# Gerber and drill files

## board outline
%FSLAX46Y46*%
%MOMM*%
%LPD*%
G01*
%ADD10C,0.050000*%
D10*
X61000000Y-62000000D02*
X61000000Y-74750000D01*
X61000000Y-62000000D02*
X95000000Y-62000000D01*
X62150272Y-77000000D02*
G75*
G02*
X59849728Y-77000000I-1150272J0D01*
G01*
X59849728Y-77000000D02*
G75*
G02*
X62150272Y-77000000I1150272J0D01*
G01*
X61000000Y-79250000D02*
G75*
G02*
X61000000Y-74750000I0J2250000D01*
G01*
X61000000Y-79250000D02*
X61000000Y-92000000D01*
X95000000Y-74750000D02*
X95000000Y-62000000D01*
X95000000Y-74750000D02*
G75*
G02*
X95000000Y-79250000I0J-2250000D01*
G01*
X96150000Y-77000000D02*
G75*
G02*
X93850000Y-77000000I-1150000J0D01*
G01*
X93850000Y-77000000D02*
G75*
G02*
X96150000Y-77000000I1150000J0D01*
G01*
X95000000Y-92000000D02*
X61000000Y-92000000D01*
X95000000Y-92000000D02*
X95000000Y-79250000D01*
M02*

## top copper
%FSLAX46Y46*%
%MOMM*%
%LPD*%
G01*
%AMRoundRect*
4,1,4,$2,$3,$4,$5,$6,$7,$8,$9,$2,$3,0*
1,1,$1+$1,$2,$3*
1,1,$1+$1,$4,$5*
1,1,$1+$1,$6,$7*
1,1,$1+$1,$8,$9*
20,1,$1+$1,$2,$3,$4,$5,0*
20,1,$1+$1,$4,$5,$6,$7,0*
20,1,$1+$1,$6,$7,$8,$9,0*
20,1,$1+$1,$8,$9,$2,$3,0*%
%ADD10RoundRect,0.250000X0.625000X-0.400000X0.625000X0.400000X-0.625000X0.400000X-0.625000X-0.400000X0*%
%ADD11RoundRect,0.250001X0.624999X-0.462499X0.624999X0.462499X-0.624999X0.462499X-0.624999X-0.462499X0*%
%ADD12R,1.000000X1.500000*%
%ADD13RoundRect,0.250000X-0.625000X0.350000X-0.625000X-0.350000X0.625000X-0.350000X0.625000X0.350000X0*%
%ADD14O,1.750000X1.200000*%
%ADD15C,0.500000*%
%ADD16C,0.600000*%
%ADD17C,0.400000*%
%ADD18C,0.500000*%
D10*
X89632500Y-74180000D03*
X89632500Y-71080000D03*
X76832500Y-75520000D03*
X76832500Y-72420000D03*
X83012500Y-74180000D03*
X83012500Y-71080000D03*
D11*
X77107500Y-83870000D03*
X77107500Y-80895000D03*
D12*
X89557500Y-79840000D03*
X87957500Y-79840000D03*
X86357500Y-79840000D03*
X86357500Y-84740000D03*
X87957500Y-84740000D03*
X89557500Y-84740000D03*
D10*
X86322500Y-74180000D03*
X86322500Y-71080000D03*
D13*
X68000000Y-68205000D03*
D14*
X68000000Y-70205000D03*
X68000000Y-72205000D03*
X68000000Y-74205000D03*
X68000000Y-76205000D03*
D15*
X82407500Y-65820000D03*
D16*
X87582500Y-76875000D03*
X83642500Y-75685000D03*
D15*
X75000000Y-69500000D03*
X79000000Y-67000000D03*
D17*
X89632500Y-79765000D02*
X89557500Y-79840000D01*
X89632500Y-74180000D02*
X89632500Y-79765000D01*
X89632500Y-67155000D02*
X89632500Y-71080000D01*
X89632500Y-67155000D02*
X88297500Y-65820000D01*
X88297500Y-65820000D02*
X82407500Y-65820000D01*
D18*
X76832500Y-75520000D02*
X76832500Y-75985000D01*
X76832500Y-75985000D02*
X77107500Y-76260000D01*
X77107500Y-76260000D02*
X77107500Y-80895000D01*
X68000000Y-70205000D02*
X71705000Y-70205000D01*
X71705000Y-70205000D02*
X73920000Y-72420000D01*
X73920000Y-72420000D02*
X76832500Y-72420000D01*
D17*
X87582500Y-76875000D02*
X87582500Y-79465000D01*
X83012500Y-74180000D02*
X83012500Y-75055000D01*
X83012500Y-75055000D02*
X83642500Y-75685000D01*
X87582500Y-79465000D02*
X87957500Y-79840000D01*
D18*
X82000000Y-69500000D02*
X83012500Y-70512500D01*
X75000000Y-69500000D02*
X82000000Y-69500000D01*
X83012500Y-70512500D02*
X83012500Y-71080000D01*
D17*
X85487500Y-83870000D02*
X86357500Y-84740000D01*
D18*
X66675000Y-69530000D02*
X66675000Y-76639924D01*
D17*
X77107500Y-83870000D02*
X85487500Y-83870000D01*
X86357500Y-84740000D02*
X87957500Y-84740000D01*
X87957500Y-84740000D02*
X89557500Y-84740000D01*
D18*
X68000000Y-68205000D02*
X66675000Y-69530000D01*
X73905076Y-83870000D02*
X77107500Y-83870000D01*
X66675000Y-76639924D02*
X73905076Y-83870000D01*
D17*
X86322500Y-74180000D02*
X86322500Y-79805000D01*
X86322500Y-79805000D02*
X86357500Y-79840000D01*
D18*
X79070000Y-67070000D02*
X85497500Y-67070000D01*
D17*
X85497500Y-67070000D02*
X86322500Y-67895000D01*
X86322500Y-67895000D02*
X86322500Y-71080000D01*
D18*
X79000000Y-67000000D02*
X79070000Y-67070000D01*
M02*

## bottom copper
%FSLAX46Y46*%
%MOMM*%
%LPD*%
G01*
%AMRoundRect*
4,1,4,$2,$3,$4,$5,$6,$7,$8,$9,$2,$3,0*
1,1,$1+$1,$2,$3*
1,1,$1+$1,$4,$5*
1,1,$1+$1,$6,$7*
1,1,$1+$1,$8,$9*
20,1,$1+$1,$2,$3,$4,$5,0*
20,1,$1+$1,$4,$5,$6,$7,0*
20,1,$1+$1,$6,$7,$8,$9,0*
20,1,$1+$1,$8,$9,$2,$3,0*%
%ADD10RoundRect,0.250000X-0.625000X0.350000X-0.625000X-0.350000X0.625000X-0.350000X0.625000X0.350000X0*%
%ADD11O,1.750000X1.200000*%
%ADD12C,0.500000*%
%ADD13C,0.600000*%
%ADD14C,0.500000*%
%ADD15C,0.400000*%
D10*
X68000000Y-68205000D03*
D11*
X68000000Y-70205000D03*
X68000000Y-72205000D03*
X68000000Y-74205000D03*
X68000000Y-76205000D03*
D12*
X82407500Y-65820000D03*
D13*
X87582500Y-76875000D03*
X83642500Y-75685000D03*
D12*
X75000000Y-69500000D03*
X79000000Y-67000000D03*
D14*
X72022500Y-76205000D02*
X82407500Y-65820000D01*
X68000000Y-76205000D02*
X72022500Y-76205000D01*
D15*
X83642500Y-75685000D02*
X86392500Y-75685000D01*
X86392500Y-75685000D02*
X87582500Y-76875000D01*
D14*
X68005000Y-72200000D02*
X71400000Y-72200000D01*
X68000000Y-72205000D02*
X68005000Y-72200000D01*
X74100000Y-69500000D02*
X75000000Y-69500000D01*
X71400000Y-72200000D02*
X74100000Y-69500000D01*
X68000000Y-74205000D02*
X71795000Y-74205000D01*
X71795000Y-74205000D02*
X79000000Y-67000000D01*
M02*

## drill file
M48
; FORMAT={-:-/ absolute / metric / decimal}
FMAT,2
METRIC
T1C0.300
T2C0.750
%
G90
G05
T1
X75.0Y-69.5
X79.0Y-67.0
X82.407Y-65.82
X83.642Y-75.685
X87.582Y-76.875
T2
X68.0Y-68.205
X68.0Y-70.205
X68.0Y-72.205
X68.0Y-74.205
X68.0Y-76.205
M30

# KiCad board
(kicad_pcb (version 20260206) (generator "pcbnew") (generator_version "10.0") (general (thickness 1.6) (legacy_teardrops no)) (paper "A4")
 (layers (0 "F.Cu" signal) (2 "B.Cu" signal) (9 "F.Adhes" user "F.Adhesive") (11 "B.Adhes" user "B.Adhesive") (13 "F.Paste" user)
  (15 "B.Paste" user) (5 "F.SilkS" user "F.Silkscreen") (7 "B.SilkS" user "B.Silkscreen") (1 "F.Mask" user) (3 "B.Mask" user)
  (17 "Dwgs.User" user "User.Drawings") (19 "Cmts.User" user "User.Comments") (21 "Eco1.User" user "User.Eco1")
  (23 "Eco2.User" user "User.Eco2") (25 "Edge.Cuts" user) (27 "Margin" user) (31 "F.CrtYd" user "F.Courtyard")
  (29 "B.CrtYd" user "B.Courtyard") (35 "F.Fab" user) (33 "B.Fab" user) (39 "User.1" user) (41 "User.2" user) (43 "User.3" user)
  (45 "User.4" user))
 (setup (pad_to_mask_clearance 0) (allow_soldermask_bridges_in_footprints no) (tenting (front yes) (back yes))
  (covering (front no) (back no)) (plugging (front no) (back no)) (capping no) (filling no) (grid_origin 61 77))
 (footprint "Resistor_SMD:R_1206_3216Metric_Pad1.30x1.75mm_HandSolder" (layer "F.Cu") (at 89.6325 72.63 90)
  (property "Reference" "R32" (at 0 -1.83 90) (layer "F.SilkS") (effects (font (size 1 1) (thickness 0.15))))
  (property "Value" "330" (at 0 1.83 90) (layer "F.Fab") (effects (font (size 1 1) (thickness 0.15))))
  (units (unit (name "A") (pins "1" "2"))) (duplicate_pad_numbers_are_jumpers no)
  (pad "1" smd roundrect (at -1.55 0 90) (size 1.3 1.75) (layers "F.Cu" "F.Mask" "F.Paste") (roundrect_rratio 0.192308)
   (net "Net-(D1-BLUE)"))
  (pad "2" smd roundrect (at 1.55 0 90) (size 1.3 1.75) (layers "F.Cu" "F.Mask" "F.Paste") (roundrect_rratio 0.192308) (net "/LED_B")))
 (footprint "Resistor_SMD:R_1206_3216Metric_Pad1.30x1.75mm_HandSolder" (layer "F.Cu") (at 76.8325 73.97 90)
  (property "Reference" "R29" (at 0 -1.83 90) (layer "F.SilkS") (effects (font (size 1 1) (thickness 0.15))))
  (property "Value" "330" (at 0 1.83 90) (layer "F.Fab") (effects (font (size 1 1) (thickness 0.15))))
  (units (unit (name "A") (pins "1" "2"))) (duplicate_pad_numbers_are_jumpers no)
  (pad "1" smd roundrect (at -1.55 0 90) (size 1.3 1.75) (layers "F.Cu" "F.Mask" "F.Paste") (roundrect_rratio 0.192308) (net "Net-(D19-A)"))
  (pad "2" smd roundrect (at 1.55 0 90) (size 1.3 1.75) (layers "F.Cu" "F.Mask" "F.Paste") (roundrect_rratio 0.192308) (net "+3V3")))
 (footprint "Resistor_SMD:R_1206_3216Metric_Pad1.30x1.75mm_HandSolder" (layer "F.Cu") (at 83.0125 72.63 90)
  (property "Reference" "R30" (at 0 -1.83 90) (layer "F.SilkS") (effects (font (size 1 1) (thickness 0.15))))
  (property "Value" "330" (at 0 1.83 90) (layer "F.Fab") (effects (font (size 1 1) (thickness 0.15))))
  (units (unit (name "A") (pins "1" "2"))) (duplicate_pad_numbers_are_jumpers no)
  (pad "1" smd roundrect (at -1.55 0 90) (size 1.3 1.75) (layers "F.Cu" "F.Mask" "F.Paste") (roundrect_rratio 0.192308) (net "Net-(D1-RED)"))
  (pad "2" smd roundrect (at 1.55 0 90) (size 1.3 1.75) (layers "F.Cu" "F.Mask" "F.Paste") (roundrect_rratio 0.192308) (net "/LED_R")))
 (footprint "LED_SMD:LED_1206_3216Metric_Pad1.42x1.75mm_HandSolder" (layer "F.Cu") (at 77.1075 82.3825 90)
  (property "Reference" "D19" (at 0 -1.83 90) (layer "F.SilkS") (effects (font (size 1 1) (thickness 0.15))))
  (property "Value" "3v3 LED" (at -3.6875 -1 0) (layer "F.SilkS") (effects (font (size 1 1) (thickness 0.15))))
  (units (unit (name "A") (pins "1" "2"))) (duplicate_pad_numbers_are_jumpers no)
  (pad "1" smd roundrect (at -1.4875 0 90) (size 1.425 1.75) (layers "F.Cu" "F.Mask" "F.Paste") (roundrect_rratio 0.175439) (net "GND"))
  (pad "2" smd roundrect (at 1.4875 0 90) (size 1.425 1.75) (layers "F.Cu" "F.Mask" "F.Paste") (roundrect_rratio 0.175439)
   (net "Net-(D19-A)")))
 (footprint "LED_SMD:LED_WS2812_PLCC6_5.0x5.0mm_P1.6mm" (layer "F.Cu") (at 87.9575 82.29 -90)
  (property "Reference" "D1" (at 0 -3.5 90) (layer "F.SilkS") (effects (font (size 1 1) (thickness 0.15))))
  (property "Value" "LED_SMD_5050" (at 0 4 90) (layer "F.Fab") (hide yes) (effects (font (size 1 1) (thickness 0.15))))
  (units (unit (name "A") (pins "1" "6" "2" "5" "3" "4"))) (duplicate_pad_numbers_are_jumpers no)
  (pad "1" smd rect (at -2.45 -1.6 270) (size 1.5 1) (layers "F.Cu" "F.Mask" "F.Paste") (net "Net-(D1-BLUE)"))
  (pad "2" smd rect (at -2.45 0 270) (size 1.5 1) (layers "F.Cu" "F.Mask" "F.Paste") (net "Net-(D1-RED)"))
  (pad "3" smd rect (at -2.45 1.6 270) (size 1.5 1) (layers "F.Cu" "F.Mask" "F.Paste") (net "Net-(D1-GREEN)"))
  (pad "4" smd rect (at 2.45 1.6 270) (size 1.5 1) (layers "F.Cu" "F.Mask" "F.Paste") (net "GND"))
  (pad "5" smd rect (at 2.45 0 270) (size 1.5 1) (layers "F.Cu" "F.Mask" "F.Paste") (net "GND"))
  (pad "6" smd rect (at 2.45 -1.6 270) (size 1.5 1) (layers "F.Cu" "F.Mask" "F.Paste") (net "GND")))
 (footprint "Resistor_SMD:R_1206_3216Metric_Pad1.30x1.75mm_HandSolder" (layer "F.Cu") (at 86.3225 72.63 90)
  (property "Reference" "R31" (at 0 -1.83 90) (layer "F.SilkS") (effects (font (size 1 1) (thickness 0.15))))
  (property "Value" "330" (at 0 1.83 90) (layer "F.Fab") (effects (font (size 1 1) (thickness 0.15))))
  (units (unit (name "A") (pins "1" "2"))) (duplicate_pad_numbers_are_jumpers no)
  (pad "1" smd roundrect (at -1.55 0 90) (size 1.3 1.75) (layers "F.Cu" "F.Mask" "F.Paste") (roundrect_rratio 0.192308)
   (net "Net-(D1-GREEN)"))
  (pad "2" smd roundrect (at 1.55 0 90) (size 1.3 1.75) (layers "F.Cu" "F.Mask" "F.Paste") (roundrect_rratio 0.192308) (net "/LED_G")))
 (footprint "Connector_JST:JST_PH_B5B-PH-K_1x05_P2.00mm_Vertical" (layer "B.Cu") (at 68 68.205 -90)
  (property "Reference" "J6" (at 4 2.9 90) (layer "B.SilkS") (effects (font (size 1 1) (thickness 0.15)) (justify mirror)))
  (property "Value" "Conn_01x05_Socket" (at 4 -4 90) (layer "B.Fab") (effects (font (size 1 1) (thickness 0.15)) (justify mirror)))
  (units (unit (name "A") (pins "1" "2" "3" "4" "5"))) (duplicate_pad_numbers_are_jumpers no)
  (pad "1" thru_hole roundrect (at 0 0 270) (size 1.2 1.75) (drill 0.75) (layers "*.Cu" "*.Mask") (remove_unused_layers no)
   (roundrect_rratio 0.208333) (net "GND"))
  (pad "2" thru_hole oval (at 2 0 270) (size 1.2 1.75) (drill 0.75) (layers "*.Cu" "*.Mask") (remove_unused_layers no) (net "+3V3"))
  (pad "3" thru_hole oval (at 4 0 270) (size 1.2 1.75) (drill 0.75) (layers "*.Cu" "*.Mask") (remove_unused_layers no) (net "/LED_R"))
  (pad "4" thru_hole oval (at 6 0 270) (size 1.2 1.75) (drill 0.75) (layers "*.Cu" "*.Mask") (remove_unused_layers no) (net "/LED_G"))
  (pad "5" thru_hole oval (at 8 0 270) (size 1.2 1.75) (drill 0.75) (layers "*.Cu" "*.Mask") (remove_unused_layers no) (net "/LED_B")))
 (gr_line (start 61 62) (end 61 74.75) (stroke (width 0.05) (type solid)) (layer "Edge.Cuts"))
 (gr_line (start 61 62) (end 95 62) (stroke (width 0.05) (type solid)) (layer "Edge.Cuts"))
 (gr_circle (center 61 77) (end 62.15 77.025) (stroke (width 0.05) (type default)) (fill no) (layer "Edge.Cuts"))
 (gr_arc (start 61 79.25) (mid 58.75 77) (end 61 74.75) (stroke (width 0.05) (type default)) (layer "Edge.Cuts"))
 (gr_line (start 61 79.25) (end 61 92) (stroke (width 0.05) (type solid)) (layer "Edge.Cuts"))
 (gr_line (start 95 74.75) (end 95 62) (stroke (width 0.05) (type solid)) (layer "Edge.Cuts"))
 (gr_arc (start 95 74.75) (mid 97.25 77) (end 95 79.25) (stroke (width 0.05) (type solid)) (layer "Edge.Cuts"))
 (gr_circle (center 95 77) (end 96.15 77) (stroke (width 0.05) (type solid)) (fill no) (layer "Edge.Cuts"))
 (gr_line (start 95 92) (end 61 92) (stroke (width 0.05) (type solid)) (layer "Edge.Cuts"))
 (gr_line (start 95 92) (end 95 79.25) (stroke (width 0.05) (type solid)) (layer "Edge.Cuts"))
 (segment (start 89.6325 79.765) (end 89.5575 79.84) (width 0.4) (layer "F.Cu") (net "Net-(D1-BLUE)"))
 (segment (start 89.6325 74.18) (end 89.6325 79.765) (width 0.4) (layer "F.Cu") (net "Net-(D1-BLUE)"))
 (segment (start 89.6325 67.155) (end 89.6325 71.08) (width 0.4) (layer "F.Cu") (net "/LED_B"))
 (segment (start 89.6325 67.155) (end 88.2975 65.82) (width 0.4) (layer "F.Cu") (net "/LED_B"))
 (segment (start 88.2975 65.82) (end 82.4075 65.82) (width 0.4) (layer "F.Cu") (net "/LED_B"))
 (via (at 82.4075 65.82) (size 0.5) (drill 0.3) (layers "F.Cu" "B.Cu") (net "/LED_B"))
 (segment (start 72.0225 76.205) (end 82.4075 65.82) (width 0.5) (layer "B.Cu") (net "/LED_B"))
 (segment (start 68 76.205) (end 72.0225 76.205) (width 0.5) (layer "B.Cu") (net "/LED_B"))
 (segment (start 76.8325 75.52) (end 76.8325 75.985) (width 0.5) (layer "F.Cu") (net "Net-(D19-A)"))
 (segment (start 76.8325 75.985) (end 77.1075 76.26) (width 0.5) (layer "F.Cu") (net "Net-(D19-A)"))
 (segment (start 77.1075 76.26) (end 77.1075 80.895) (width 0.5) (layer "F.Cu") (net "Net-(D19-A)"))
 (segment (start 68 70.205) (end 71.705 70.205) (width 0.5) (layer "F.Cu") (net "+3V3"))
 (segment (start 71.705 70.205) (end 73.92 72.42) (width 0.5) (layer "F.Cu") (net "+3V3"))
 (segment (start 73.92 72.42) (end 76.8325 72.42) (width 0.5) (layer "F.Cu") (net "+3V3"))
 (segment (start 87.5825 76.875) (end 87.5825 79.465) (width 0.4) (layer "F.Cu") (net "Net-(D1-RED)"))
 (segment (start 83.0125 74.18) (end 83.0125 75.055) (width 0.4) (layer "F.Cu") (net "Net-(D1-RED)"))
 (segment (start 83.0125 75.055) (end 83.6425 75.685) (width 0.4) (layer "F.Cu") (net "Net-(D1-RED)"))
 (segment (start 87.5825 79.465) (end 87.9575 79.84) (width 0.4) (layer "F.Cu") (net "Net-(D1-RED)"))
 (via (at 87.5825 76.875) (size 0.6) (drill 0.3) (layers "F.Cu" "B.Cu") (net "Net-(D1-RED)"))
 (via (at 83.6425 75.685) (size 0.6) (drill 0.3) (layers "F.Cu" "B.Cu") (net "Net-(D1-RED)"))
 (segment (start 83.6425 75.685) (end 86.3925 75.685) (width 0.4) (layer "B.Cu") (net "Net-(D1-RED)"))
 (segment (start 86.3925 75.685) (end 87.5825 76.875) (width 0.4) (layer "B.Cu") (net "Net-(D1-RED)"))
 (segment (start 82 69.5) (end 83.0125 70.5125) (width 0.5) (layer "F.Cu") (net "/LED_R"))
 (segment (start 75 69.5) (end 82 69.5) (width 0.5) (layer "F.Cu") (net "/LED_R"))
 (segment (start 83.0125 70.5125) (end 83.0125 71.08) (width 0.5) (layer "F.Cu") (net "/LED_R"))
 (via (at 75 69.5) (size 0.5) (drill 0.3) (layers "F.Cu" "B.Cu") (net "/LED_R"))
 (segment (start 68.005 72.2) (end 71.4 72.2) (width 0.5) (layer "B.Cu") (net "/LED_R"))
 (segment (start 68 72.205) (end 68.005 72.2) (width 0.5) (layer "B.Cu") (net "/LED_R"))
 (segment (start 74.1 69.5) (end 75 69.5) (width 0.5) (layer "B.Cu") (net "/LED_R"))
 (segment (start 71.4 72.2) (end 74.1 69.5) (width 0.5) (layer "B.Cu") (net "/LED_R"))
 (segment (start 85.4875 83.87) (end 86.3575 84.74) (width 0.4) (layer "F.Cu") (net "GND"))
 (segment (start 66.675 69.53) (end 66.675 76.639924) (width 0.5) (layer "F.Cu") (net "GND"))
 (segment (start 77.1075 83.87) (end 85.4875 83.87) (width 0.4) (layer "F.Cu") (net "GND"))
 (segment (start 86.3575 84.74) (end 87.9575 84.74) (width 0.4) (layer "F.Cu") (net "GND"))
 (segment (start 87.9575 84.74) (end 89.5575 84.74) (width 0.4) (layer "F.Cu") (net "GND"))
 (segment (start 68 68.205) (end 66.675 69.53) (width 0.5) (layer "F.Cu") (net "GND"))
 (segment (start 73.905076 83.87) (end 77.1075 83.87) (width 0.5) (layer "F.Cu") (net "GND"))
 (segment (start 66.675 76.639924) (end 73.905076 83.87) (width 0.5) (layer "F.Cu") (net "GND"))
 (segment (start 86.3225 74.18) (end 86.3225 79.805) (width 0.4) (layer "F.Cu") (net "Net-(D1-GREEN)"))
 (segment (start 86.3225 79.805) (end 86.3575 79.84) (width 0.4) (layer "F.Cu") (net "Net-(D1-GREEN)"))
 (segment (start 79.07 67.07) (end 85.4975 67.07) (width 0.5) (layer "F.Cu") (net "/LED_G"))
 (segment (start 85.4975 67.07) (end 86.3225 67.895) (width 0.4) (layer "F.Cu") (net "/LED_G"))
 (segment (start 86.3225 67.895) (end 86.3225 71.08) (width 0.4) (layer "F.Cu") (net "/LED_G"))
 (segment (start 79 67) (end 79.07 67.07) (width 0.5) (layer "F.Cu") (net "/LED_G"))
 (via (at 79 67) (size 0.5) (drill 0.3) (layers "F.Cu" "B.Cu") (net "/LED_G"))
 (segment (start 68 74.205) (end 71.795 74.205) (width 0.5) (layer "B.Cu") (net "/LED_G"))
 (segment (start 71.795 74.205) (end 79 67) (width 0.5) (layer "B.Cu") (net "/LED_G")))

